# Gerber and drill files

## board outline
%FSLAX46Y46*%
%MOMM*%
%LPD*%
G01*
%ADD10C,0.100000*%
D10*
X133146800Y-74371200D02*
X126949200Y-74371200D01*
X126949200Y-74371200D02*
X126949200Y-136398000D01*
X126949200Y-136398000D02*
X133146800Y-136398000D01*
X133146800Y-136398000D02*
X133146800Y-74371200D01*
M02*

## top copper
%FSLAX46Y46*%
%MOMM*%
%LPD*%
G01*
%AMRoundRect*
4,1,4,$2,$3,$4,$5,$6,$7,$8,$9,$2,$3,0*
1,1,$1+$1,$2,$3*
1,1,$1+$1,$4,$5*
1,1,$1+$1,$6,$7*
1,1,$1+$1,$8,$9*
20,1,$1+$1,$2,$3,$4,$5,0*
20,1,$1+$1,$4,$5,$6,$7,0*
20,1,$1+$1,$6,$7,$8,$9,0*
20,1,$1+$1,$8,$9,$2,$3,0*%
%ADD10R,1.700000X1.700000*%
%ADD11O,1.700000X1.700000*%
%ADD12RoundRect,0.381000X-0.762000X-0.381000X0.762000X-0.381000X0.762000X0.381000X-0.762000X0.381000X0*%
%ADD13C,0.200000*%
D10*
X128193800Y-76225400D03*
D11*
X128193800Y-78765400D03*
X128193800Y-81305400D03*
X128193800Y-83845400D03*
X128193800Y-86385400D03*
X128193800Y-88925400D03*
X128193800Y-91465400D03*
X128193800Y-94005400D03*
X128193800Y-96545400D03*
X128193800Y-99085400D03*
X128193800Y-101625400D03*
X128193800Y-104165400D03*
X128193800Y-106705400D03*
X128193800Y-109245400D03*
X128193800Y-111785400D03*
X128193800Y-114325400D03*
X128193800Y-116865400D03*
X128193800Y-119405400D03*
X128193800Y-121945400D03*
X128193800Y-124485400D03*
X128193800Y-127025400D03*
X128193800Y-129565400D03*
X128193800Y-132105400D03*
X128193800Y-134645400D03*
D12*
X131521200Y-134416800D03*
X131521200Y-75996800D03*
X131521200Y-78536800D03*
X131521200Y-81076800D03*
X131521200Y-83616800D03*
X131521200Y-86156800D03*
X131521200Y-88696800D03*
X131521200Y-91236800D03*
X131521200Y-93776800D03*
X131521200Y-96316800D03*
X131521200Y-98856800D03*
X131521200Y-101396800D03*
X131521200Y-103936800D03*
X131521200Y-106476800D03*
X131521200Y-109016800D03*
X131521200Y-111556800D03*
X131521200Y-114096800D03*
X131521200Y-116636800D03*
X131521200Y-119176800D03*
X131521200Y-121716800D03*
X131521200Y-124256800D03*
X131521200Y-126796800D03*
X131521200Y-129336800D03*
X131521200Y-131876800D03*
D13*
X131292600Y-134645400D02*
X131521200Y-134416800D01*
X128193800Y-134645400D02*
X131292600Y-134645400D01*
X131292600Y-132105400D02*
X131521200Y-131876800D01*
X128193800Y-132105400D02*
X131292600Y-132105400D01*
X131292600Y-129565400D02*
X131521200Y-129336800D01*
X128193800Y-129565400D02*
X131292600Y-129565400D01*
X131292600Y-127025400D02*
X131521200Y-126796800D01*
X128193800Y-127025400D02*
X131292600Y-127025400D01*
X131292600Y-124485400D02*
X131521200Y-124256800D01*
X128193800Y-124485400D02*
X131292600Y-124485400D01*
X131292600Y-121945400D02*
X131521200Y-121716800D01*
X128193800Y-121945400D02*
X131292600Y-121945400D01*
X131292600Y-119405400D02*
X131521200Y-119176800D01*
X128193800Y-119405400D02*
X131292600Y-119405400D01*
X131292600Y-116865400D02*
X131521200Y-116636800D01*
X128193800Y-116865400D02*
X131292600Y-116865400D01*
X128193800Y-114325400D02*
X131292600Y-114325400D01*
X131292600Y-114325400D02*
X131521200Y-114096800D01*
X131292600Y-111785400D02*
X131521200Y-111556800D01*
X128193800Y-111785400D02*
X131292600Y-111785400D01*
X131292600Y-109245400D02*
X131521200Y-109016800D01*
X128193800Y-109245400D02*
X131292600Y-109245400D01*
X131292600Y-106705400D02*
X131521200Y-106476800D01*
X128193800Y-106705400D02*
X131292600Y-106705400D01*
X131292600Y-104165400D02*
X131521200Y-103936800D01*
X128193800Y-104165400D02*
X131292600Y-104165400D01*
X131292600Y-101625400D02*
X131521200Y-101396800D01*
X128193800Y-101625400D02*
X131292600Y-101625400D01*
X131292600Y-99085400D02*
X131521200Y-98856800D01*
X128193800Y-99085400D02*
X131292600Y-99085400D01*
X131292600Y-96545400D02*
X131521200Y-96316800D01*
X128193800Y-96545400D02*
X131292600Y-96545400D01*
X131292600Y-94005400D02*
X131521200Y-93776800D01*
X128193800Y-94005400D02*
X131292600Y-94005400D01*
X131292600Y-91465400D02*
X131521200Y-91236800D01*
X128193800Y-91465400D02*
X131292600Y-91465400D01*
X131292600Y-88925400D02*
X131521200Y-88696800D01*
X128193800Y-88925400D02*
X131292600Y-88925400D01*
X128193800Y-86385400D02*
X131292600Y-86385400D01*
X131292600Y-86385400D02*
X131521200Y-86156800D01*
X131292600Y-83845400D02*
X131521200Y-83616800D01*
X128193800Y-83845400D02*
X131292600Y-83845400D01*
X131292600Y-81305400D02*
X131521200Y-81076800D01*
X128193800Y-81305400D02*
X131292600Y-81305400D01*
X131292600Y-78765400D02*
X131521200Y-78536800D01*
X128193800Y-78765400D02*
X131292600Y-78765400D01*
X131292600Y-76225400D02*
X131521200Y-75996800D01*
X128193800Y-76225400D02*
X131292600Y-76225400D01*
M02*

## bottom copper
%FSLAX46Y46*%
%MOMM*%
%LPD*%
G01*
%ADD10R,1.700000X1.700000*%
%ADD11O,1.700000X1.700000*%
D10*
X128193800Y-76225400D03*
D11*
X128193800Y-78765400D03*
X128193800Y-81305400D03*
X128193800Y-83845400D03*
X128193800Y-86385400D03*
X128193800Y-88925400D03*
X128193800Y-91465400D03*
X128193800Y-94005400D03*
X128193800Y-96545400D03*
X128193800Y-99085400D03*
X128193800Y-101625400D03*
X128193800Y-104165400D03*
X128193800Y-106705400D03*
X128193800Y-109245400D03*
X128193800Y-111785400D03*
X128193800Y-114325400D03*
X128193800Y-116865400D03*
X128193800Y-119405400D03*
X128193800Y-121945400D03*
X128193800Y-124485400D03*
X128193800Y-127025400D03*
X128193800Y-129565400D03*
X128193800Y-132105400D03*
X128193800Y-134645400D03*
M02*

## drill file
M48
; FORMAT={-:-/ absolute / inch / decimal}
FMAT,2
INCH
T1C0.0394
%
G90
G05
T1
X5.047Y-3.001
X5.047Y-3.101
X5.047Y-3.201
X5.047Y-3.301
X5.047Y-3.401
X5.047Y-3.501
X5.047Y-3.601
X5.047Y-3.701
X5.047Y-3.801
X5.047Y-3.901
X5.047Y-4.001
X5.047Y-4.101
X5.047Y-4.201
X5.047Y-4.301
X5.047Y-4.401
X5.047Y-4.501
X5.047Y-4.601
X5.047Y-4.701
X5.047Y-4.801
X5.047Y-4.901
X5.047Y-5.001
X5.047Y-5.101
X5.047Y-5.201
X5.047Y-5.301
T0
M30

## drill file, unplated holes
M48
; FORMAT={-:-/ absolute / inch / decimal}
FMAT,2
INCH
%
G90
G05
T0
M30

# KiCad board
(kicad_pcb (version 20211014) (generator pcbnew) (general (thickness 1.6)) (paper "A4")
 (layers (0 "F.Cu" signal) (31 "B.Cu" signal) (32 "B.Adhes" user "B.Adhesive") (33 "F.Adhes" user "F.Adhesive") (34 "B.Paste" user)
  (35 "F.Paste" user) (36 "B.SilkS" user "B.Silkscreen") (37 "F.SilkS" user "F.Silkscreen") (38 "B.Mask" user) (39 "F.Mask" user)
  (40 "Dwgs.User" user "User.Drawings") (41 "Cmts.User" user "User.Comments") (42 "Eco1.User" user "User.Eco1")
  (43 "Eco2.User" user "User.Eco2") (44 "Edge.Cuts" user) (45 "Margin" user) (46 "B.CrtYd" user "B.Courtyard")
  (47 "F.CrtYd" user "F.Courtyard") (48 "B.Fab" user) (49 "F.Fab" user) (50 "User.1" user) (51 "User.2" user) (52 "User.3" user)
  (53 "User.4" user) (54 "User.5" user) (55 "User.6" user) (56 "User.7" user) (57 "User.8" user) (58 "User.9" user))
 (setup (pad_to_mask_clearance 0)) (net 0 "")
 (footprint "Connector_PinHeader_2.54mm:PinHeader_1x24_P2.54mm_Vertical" (layer "F.Cu") (at 128.1938 76.2254)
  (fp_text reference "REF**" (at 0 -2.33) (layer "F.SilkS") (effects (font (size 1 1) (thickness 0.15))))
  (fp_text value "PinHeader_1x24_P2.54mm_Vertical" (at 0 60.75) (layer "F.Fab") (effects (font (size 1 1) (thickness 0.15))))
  (pad "1" thru_hole rect (at 0 0) (size 1.7 1.7) (drill 1) (layers *.Cu *.Mask))
  (pad "2" thru_hole oval (at 0 2.54) (size 1.7 1.7) (drill 1) (layers *.Cu *.Mask))
  (pad "3" thru_hole oval (at 0 5.08) (size 1.7 1.7) (drill 1) (layers *.Cu *.Mask))
  (pad "4" thru_hole oval (at 0 7.62) (size 1.7 1.7) (drill 1) (layers *.Cu *.Mask))
  (pad "5" thru_hole oval (at 0 10.16) (size 1.7 1.7) (drill 1) (layers *.Cu *.Mask))
  (pad "6" thru_hole oval (at 0 12.7) (size 1.7 1.7) (drill 1) (layers *.Cu *.Mask))
  (pad "7" thru_hole oval (at 0 15.24) (size 1.7 1.7) (drill 1) (layers *.Cu *.Mask))
  (pad "8" thru_hole oval (at 0 17.78) (size 1.7 1.7) (drill 1) (layers *.Cu *.Mask))
  (pad "9" thru_hole oval (at 0 20.32) (size 1.7 1.7) (drill 1) (layers *.Cu *.Mask))
  (pad "10" thru_hole oval (at 0 22.86) (size 1.7 1.7) (drill 1) (layers *.Cu *.Mask))
  (pad "11" thru_hole oval (at 0 25.4) (size 1.7 1.7) (drill 1) (layers *.Cu *.Mask))
  (pad "12" thru_hole oval (at 0 27.94) (size 1.7 1.7) (drill 1) (layers *.Cu *.Mask))
  (pad "13" thru_hole oval (at 0 30.48) (size 1.7 1.7) (drill 1) (layers *.Cu *.Mask))
  (pad "14" thru_hole oval (at 0 33.02) (size 1.7 1.7) (drill 1) (layers *.Cu *.Mask))
  (pad "15" thru_hole oval (at 0 35.56) (size 1.7 1.7) (drill 1) (layers *.Cu *.Mask))
  (pad "16" thru_hole oval (at 0 38.1) (size 1.7 1.7) (drill 1) (layers *.Cu *.Mask))
  (pad "17" thru_hole oval (at 0 40.64) (size 1.7 1.7) (drill 1) (layers *.Cu *.Mask))
  (pad "18" thru_hole oval (at 0 43.18) (size 1.7 1.7) (drill 1) (layers *.Cu *.Mask))
  (pad "19" thru_hole oval (at 0 45.72) (size 1.7 1.7) (drill 1) (layers *.Cu *.Mask))
  (pad "20" thru_hole oval (at 0 48.26) (size 1.7 1.7) (drill 1) (layers *.Cu *.Mask))
  (pad "21" thru_hole oval (at 0 50.8) (size 1.7 1.7) (drill 1) (layers *.Cu *.Mask))
  (pad "22" thru_hole oval (at 0 53.34) (size 1.7 1.7) (drill 1) (layers *.Cu *.Mask))
  (pad "23" thru_hole oval (at 0 55.88) (size 1.7 1.7) (drill 1) (layers *.Cu *.Mask))
  (pad "24" thru_hole oval (at 0 58.42) (size 1.7 1.7) (drill 1) (layers *.Cu *.Mask)))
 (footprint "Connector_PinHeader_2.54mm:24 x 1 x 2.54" (layer "F.Cu") (at 131.5212 75.9968)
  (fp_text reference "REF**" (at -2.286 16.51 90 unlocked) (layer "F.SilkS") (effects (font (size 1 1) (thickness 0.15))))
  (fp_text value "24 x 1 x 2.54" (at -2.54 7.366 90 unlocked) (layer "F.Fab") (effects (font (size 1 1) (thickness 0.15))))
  (pad "2" smd roundrect (at 0 0) (size 2.286 1.524) (layers "F.Cu" "F.Paste" "F.Mask") (roundrect_rratio 0.25))
  (pad "3" smd roundrect (at 0 2.54) (size 2.286 1.524) (layers "F.Cu" "F.Paste" "F.Mask") (roundrect_rratio 0.25))
  (pad "4" smd roundrect (at 0 5.08) (size 2.286 1.524) (layers "F.Cu" "F.Paste" "F.Mask") (roundrect_rratio 0.25))
  (pad "5" smd roundrect (at 0 7.62) (size 2.286 1.524) (layers "F.Cu" "F.Paste" "F.Mask") (roundrect_rratio 0.25))
  (pad "6" smd roundrect (at 0 10.16) (size 2.286 1.524) (layers "F.Cu" "F.Paste" "F.Mask") (roundrect_rratio 0.25))
  (pad "7" smd roundrect (at 0 12.7) (size 2.286 1.524) (layers "F.Cu" "F.Paste" "F.Mask") (roundrect_rratio 0.25))
  (pad "8" smd roundrect (at 0 15.24) (size 2.286 1.524) (layers "F.Cu" "F.Paste" "F.Mask") (roundrect_rratio 0.25))
  (pad "9" smd roundrect (at 0 17.78) (size 2.286 1.524) (layers "F.Cu" "F.Paste" "F.Mask") (roundrect_rratio 0.25))
  (pad "10" smd roundrect (at 0 20.32) (size 2.286 1.524) (layers "F.Cu" "F.Paste" "F.Mask") (roundrect_rratio 0.25))
  (pad "11" smd roundrect (at 0 22.86) (size 2.286 1.524) (layers "F.Cu" "F.Paste" "F.Mask") (roundrect_rratio 0.25))
  (pad "12" smd roundrect (at 0 25.4) (size 2.286 1.524) (layers "F.Cu" "F.Paste" "F.Mask") (roundrect_rratio 0.25))
  (pad "13" smd roundrect (at 0 27.94) (size 2.286 1.524) (layers "F.Cu" "F.Paste" "F.Mask") (roundrect_rratio 0.25))
  (pad "14" smd roundrect (at 0 30.48) (size 2.286 1.524) (layers "F.Cu" "F.Paste" "F.Mask") (roundrect_rratio 0.25))
  (pad "15" smd roundrect (at 0 33.02) (size 2.286 1.524) (layers "F.Cu" "F.Paste" "F.Mask") (roundrect_rratio 0.25))
  (pad "16" smd roundrect (at 0 35.56) (size 2.286 1.524) (layers "F.Cu" "F.Paste" "F.Mask") (roundrect_rratio 0.25))
  (pad "17" smd roundrect (at 0 38.1) (size 2.286 1.524) (layers "F.Cu" "F.Paste" "F.Mask") (roundrect_rratio 0.25))
  (pad "18" smd roundrect (at 0 40.64) (size 2.286 1.524) (layers "F.Cu" "F.Paste" "F.Mask") (roundrect_rratio 0.25))
  (pad "19" smd roundrect (at 0 43.18) (size 2.286 1.524) (layers "F.Cu" "F.Paste" "F.Mask") (roundrect_rratio 0.25))
  (pad "20" smd roundrect (at 0 45.72) (size 2.286 1.524) (layers "F.Cu" "F.Paste" "F.Mask") (roundrect_rratio 0.25))
  (pad "21" smd roundrect (at 0 48.26) (size 2.286 1.524) (layers "F.Cu" "F.Paste" "F.Mask") (roundrect_rratio 0.25))
  (pad "22" smd roundrect (at 0 50.8) (size 2.286 1.524) (layers "F.Cu" "F.Paste" "F.Mask") (roundrect_rratio 0.25))
  (pad "23" smd roundrect (at 0 53.34) (size 2.286 1.524) (layers "F.Cu" "F.Paste" "F.Mask") (roundrect_rratio 0.25))
  (pad "24" smd roundrect (at 0 55.88) (size 2.286 1.524) (layers "F.Cu" "F.Paste" "F.Mask") (roundrect_rratio 0.25))
  (pad "25" smd roundrect (at 0 58.42) (size 2.286 1.524) (layers "F.Cu" "F.Paste" "F.Mask") (roundrect_rratio 0.25)))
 (gr_rect (start 133.1468 74.3712) (end 126.9492 136.398) (layer "Edge.Cuts") (width 0.1) (fill none))
 (segment (start 128.1938 109.2454) (end 131.2926 109.2454) (width 0.2) (layer "F.Cu") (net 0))
 (segment (start 128.1938 129.5654) (end 131.2926 129.5654) (width 0.2) (layer "F.Cu") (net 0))
 (segment (start 131.2926 114.3254) (end 131.5212 114.0968) (width 0.2) (layer "F.Cu") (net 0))
 (segment (start 128.1938 119.4054) (end 131.2926 119.4054) (width 0.2) (layer "F.Cu") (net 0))
 (segment (start 128.1938 81.3054) (end 131.2926 81.3054) (width 0.2) (layer "F.Cu") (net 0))
 (segment (start 128.1938 134.6454) (end 131.2926 134.6454) (width 0.2) (layer "F.Cu") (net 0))
 (segment (start 128.1938 101.6254) (end 131.2926 101.6254) (width 0.2) (layer "F.Cu") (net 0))
 (segment (start 131.2926 124.4854) (end 131.5212 124.2568) (width 0.2) (layer "F.Cu") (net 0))
 (segment (start 128.1938 116.8654) (end 131.2926 116.8654) (width 0.2) (layer "F.Cu") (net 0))
 (segment (start 128.1938 132.1054) (end 131.2926 132.1054) (width 0.2) (layer "F.Cu") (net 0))
 (segment (start 128.1938 88.9254) (end 131.2926 88.9254) (width 0.2) (layer "F.Cu") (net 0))
 (segment (start 131.2926 104.1654) (end 131.5212 103.9368) (width 0.2) (layer "F.Cu") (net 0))
 (segment (start 128.1938 121.9454) (end 131.2926 121.9454) (width 0.2) (layer "F.Cu") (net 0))
 (segment (start 128.1938 78.7654) (end 131.2926 78.7654) (width 0.2) (layer "F.Cu") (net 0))
 (segment (start 128.1938 106.7054) (end 131.2926 106.7054) (width 0.2) (layer "F.Cu") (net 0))
 (segment (start 128.1938 76.2254) (end 131.2926 76.2254) (width 0.2) (layer "F.Cu") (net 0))
 (segment (start 131.2926 111.7854) (end 131.5212 111.5568) (width 0.2) (layer "F.Cu") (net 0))
 (segment (start 131.2926 101.6254) (end 131.5212 101.3968) (width 0.2) (layer "F.Cu") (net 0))
 (segment (start 131.2926 76.2254) (end 131.5212 75.9968) (width 0.2) (layer "F.Cu") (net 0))
 (segment (start 128.1938 111.7854) (end 131.2926 111.7854) (width 0.2) (layer "F.Cu") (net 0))
 (segment (start 128.1938 104.1654) (end 131.2926 104.1654) (width 0.2) (layer "F.Cu") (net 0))
 (segment (start 128.1938 94.0054) (end 131.2926 94.0054) (width 0.2) (layer "F.Cu") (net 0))
 (segment (start 131.2926 96.5454) (end 131.5212 96.3168) (width 0.2) (layer "F.Cu") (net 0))
 (segment (start 131.2926 99.0854) (end 131.5212 98.8568) (width 0.2) (layer "F.Cu") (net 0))
 (segment (start 128.1938 83.8454) (end 131.2926 83.8454) (width 0.2) (layer "F.Cu") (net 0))
 (segment (start 128.1938 114.3254) (end 131.2926 114.3254) (width 0.2) (layer "F.Cu") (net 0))
 (segment (start 131.2926 132.1054) (end 131.5212 131.8768) (width 0.2) (layer "F.Cu") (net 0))
 (segment (start 128.1938 99.0854) (end 131.2926 99.0854) (width 0.2) (layer "F.Cu") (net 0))
 (segment (start 128.1938 96.5454) (end 131.2926 96.5454) (width 0.2) (layer "F.Cu") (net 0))
 (segment (start 131.2926 119.4054) (end 131.5212 119.1768) (width 0.2) (layer "F.Cu") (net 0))
 (segment (start 131.2926 94.0054) (end 131.5212 93.7768) (width 0.2) (layer "F.Cu") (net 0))
 (segment (start 131.2926 121.9454) (end 131.5212 121.7168) (width 0.2) (layer "F.Cu") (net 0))
 (segment (start 128.1938 127.0254) (end 131.2926 127.0254) (width 0.2) (layer "F.Cu") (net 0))
 (segment (start 131.2926 106.7054) (end 131.5212 106.4768) (width 0.2) (layer "F.Cu") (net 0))
 (segment (start 131.2926 91.4654) (end 131.5212 91.2368) (width 0.2) (layer "F.Cu") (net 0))
 (segment (start 131.2926 83.8454) (end 131.5212 83.6168) (width 0.2) (layer "F.Cu") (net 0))
 (segment (start 131.2926 134.6454) (end 131.5212 134.4168) (width 0.2) (layer "F.Cu") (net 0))
 (segment (start 131.2926 116.8654) (end 131.5212 116.6368) (width 0.2) (layer "F.Cu") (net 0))
 (segment (start 131.2926 86.3854) (end 131.5212 86.1568) (width 0.2) (layer "F.Cu") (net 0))
 (segment (start 128.1938 91.4654) (end 131.2926 91.4654) (width 0.2) (layer "F.Cu") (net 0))
 (segment (start 131.2926 127.0254) (end 131.5212 126.7968) (width 0.2) (layer "F.Cu") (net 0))
 (segment (start 131.2926 88.9254) (end 131.5212 88.6968) (width 0.2) (layer "F.Cu") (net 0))
 (segment (start 131.2926 81.3054) (end 131.5212 81.0768) (width 0.2) (layer "F.Cu") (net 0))
 (segment (start 131.2926 78.7654) (end 131.5212 78.5368) (width 0.2) (layer "F.Cu") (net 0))
 (segment (start 131.2926 109.2454) (end 131.5212 109.0168) (width 0.2) (layer "F.Cu") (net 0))
 (segment (start 128.1938 124.4854) (end 131.2926 124.4854) (width 0.2) (layer "F.Cu") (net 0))
 (segment (start 131.2926 129.5654) (end 131.5212 129.3368) (width 0.2) (layer "F.Cu") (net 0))
 (segment (start 128.1938 86.3854) (end 131.2926 86.3854) (width 0.2) (layer "F.Cu") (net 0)))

